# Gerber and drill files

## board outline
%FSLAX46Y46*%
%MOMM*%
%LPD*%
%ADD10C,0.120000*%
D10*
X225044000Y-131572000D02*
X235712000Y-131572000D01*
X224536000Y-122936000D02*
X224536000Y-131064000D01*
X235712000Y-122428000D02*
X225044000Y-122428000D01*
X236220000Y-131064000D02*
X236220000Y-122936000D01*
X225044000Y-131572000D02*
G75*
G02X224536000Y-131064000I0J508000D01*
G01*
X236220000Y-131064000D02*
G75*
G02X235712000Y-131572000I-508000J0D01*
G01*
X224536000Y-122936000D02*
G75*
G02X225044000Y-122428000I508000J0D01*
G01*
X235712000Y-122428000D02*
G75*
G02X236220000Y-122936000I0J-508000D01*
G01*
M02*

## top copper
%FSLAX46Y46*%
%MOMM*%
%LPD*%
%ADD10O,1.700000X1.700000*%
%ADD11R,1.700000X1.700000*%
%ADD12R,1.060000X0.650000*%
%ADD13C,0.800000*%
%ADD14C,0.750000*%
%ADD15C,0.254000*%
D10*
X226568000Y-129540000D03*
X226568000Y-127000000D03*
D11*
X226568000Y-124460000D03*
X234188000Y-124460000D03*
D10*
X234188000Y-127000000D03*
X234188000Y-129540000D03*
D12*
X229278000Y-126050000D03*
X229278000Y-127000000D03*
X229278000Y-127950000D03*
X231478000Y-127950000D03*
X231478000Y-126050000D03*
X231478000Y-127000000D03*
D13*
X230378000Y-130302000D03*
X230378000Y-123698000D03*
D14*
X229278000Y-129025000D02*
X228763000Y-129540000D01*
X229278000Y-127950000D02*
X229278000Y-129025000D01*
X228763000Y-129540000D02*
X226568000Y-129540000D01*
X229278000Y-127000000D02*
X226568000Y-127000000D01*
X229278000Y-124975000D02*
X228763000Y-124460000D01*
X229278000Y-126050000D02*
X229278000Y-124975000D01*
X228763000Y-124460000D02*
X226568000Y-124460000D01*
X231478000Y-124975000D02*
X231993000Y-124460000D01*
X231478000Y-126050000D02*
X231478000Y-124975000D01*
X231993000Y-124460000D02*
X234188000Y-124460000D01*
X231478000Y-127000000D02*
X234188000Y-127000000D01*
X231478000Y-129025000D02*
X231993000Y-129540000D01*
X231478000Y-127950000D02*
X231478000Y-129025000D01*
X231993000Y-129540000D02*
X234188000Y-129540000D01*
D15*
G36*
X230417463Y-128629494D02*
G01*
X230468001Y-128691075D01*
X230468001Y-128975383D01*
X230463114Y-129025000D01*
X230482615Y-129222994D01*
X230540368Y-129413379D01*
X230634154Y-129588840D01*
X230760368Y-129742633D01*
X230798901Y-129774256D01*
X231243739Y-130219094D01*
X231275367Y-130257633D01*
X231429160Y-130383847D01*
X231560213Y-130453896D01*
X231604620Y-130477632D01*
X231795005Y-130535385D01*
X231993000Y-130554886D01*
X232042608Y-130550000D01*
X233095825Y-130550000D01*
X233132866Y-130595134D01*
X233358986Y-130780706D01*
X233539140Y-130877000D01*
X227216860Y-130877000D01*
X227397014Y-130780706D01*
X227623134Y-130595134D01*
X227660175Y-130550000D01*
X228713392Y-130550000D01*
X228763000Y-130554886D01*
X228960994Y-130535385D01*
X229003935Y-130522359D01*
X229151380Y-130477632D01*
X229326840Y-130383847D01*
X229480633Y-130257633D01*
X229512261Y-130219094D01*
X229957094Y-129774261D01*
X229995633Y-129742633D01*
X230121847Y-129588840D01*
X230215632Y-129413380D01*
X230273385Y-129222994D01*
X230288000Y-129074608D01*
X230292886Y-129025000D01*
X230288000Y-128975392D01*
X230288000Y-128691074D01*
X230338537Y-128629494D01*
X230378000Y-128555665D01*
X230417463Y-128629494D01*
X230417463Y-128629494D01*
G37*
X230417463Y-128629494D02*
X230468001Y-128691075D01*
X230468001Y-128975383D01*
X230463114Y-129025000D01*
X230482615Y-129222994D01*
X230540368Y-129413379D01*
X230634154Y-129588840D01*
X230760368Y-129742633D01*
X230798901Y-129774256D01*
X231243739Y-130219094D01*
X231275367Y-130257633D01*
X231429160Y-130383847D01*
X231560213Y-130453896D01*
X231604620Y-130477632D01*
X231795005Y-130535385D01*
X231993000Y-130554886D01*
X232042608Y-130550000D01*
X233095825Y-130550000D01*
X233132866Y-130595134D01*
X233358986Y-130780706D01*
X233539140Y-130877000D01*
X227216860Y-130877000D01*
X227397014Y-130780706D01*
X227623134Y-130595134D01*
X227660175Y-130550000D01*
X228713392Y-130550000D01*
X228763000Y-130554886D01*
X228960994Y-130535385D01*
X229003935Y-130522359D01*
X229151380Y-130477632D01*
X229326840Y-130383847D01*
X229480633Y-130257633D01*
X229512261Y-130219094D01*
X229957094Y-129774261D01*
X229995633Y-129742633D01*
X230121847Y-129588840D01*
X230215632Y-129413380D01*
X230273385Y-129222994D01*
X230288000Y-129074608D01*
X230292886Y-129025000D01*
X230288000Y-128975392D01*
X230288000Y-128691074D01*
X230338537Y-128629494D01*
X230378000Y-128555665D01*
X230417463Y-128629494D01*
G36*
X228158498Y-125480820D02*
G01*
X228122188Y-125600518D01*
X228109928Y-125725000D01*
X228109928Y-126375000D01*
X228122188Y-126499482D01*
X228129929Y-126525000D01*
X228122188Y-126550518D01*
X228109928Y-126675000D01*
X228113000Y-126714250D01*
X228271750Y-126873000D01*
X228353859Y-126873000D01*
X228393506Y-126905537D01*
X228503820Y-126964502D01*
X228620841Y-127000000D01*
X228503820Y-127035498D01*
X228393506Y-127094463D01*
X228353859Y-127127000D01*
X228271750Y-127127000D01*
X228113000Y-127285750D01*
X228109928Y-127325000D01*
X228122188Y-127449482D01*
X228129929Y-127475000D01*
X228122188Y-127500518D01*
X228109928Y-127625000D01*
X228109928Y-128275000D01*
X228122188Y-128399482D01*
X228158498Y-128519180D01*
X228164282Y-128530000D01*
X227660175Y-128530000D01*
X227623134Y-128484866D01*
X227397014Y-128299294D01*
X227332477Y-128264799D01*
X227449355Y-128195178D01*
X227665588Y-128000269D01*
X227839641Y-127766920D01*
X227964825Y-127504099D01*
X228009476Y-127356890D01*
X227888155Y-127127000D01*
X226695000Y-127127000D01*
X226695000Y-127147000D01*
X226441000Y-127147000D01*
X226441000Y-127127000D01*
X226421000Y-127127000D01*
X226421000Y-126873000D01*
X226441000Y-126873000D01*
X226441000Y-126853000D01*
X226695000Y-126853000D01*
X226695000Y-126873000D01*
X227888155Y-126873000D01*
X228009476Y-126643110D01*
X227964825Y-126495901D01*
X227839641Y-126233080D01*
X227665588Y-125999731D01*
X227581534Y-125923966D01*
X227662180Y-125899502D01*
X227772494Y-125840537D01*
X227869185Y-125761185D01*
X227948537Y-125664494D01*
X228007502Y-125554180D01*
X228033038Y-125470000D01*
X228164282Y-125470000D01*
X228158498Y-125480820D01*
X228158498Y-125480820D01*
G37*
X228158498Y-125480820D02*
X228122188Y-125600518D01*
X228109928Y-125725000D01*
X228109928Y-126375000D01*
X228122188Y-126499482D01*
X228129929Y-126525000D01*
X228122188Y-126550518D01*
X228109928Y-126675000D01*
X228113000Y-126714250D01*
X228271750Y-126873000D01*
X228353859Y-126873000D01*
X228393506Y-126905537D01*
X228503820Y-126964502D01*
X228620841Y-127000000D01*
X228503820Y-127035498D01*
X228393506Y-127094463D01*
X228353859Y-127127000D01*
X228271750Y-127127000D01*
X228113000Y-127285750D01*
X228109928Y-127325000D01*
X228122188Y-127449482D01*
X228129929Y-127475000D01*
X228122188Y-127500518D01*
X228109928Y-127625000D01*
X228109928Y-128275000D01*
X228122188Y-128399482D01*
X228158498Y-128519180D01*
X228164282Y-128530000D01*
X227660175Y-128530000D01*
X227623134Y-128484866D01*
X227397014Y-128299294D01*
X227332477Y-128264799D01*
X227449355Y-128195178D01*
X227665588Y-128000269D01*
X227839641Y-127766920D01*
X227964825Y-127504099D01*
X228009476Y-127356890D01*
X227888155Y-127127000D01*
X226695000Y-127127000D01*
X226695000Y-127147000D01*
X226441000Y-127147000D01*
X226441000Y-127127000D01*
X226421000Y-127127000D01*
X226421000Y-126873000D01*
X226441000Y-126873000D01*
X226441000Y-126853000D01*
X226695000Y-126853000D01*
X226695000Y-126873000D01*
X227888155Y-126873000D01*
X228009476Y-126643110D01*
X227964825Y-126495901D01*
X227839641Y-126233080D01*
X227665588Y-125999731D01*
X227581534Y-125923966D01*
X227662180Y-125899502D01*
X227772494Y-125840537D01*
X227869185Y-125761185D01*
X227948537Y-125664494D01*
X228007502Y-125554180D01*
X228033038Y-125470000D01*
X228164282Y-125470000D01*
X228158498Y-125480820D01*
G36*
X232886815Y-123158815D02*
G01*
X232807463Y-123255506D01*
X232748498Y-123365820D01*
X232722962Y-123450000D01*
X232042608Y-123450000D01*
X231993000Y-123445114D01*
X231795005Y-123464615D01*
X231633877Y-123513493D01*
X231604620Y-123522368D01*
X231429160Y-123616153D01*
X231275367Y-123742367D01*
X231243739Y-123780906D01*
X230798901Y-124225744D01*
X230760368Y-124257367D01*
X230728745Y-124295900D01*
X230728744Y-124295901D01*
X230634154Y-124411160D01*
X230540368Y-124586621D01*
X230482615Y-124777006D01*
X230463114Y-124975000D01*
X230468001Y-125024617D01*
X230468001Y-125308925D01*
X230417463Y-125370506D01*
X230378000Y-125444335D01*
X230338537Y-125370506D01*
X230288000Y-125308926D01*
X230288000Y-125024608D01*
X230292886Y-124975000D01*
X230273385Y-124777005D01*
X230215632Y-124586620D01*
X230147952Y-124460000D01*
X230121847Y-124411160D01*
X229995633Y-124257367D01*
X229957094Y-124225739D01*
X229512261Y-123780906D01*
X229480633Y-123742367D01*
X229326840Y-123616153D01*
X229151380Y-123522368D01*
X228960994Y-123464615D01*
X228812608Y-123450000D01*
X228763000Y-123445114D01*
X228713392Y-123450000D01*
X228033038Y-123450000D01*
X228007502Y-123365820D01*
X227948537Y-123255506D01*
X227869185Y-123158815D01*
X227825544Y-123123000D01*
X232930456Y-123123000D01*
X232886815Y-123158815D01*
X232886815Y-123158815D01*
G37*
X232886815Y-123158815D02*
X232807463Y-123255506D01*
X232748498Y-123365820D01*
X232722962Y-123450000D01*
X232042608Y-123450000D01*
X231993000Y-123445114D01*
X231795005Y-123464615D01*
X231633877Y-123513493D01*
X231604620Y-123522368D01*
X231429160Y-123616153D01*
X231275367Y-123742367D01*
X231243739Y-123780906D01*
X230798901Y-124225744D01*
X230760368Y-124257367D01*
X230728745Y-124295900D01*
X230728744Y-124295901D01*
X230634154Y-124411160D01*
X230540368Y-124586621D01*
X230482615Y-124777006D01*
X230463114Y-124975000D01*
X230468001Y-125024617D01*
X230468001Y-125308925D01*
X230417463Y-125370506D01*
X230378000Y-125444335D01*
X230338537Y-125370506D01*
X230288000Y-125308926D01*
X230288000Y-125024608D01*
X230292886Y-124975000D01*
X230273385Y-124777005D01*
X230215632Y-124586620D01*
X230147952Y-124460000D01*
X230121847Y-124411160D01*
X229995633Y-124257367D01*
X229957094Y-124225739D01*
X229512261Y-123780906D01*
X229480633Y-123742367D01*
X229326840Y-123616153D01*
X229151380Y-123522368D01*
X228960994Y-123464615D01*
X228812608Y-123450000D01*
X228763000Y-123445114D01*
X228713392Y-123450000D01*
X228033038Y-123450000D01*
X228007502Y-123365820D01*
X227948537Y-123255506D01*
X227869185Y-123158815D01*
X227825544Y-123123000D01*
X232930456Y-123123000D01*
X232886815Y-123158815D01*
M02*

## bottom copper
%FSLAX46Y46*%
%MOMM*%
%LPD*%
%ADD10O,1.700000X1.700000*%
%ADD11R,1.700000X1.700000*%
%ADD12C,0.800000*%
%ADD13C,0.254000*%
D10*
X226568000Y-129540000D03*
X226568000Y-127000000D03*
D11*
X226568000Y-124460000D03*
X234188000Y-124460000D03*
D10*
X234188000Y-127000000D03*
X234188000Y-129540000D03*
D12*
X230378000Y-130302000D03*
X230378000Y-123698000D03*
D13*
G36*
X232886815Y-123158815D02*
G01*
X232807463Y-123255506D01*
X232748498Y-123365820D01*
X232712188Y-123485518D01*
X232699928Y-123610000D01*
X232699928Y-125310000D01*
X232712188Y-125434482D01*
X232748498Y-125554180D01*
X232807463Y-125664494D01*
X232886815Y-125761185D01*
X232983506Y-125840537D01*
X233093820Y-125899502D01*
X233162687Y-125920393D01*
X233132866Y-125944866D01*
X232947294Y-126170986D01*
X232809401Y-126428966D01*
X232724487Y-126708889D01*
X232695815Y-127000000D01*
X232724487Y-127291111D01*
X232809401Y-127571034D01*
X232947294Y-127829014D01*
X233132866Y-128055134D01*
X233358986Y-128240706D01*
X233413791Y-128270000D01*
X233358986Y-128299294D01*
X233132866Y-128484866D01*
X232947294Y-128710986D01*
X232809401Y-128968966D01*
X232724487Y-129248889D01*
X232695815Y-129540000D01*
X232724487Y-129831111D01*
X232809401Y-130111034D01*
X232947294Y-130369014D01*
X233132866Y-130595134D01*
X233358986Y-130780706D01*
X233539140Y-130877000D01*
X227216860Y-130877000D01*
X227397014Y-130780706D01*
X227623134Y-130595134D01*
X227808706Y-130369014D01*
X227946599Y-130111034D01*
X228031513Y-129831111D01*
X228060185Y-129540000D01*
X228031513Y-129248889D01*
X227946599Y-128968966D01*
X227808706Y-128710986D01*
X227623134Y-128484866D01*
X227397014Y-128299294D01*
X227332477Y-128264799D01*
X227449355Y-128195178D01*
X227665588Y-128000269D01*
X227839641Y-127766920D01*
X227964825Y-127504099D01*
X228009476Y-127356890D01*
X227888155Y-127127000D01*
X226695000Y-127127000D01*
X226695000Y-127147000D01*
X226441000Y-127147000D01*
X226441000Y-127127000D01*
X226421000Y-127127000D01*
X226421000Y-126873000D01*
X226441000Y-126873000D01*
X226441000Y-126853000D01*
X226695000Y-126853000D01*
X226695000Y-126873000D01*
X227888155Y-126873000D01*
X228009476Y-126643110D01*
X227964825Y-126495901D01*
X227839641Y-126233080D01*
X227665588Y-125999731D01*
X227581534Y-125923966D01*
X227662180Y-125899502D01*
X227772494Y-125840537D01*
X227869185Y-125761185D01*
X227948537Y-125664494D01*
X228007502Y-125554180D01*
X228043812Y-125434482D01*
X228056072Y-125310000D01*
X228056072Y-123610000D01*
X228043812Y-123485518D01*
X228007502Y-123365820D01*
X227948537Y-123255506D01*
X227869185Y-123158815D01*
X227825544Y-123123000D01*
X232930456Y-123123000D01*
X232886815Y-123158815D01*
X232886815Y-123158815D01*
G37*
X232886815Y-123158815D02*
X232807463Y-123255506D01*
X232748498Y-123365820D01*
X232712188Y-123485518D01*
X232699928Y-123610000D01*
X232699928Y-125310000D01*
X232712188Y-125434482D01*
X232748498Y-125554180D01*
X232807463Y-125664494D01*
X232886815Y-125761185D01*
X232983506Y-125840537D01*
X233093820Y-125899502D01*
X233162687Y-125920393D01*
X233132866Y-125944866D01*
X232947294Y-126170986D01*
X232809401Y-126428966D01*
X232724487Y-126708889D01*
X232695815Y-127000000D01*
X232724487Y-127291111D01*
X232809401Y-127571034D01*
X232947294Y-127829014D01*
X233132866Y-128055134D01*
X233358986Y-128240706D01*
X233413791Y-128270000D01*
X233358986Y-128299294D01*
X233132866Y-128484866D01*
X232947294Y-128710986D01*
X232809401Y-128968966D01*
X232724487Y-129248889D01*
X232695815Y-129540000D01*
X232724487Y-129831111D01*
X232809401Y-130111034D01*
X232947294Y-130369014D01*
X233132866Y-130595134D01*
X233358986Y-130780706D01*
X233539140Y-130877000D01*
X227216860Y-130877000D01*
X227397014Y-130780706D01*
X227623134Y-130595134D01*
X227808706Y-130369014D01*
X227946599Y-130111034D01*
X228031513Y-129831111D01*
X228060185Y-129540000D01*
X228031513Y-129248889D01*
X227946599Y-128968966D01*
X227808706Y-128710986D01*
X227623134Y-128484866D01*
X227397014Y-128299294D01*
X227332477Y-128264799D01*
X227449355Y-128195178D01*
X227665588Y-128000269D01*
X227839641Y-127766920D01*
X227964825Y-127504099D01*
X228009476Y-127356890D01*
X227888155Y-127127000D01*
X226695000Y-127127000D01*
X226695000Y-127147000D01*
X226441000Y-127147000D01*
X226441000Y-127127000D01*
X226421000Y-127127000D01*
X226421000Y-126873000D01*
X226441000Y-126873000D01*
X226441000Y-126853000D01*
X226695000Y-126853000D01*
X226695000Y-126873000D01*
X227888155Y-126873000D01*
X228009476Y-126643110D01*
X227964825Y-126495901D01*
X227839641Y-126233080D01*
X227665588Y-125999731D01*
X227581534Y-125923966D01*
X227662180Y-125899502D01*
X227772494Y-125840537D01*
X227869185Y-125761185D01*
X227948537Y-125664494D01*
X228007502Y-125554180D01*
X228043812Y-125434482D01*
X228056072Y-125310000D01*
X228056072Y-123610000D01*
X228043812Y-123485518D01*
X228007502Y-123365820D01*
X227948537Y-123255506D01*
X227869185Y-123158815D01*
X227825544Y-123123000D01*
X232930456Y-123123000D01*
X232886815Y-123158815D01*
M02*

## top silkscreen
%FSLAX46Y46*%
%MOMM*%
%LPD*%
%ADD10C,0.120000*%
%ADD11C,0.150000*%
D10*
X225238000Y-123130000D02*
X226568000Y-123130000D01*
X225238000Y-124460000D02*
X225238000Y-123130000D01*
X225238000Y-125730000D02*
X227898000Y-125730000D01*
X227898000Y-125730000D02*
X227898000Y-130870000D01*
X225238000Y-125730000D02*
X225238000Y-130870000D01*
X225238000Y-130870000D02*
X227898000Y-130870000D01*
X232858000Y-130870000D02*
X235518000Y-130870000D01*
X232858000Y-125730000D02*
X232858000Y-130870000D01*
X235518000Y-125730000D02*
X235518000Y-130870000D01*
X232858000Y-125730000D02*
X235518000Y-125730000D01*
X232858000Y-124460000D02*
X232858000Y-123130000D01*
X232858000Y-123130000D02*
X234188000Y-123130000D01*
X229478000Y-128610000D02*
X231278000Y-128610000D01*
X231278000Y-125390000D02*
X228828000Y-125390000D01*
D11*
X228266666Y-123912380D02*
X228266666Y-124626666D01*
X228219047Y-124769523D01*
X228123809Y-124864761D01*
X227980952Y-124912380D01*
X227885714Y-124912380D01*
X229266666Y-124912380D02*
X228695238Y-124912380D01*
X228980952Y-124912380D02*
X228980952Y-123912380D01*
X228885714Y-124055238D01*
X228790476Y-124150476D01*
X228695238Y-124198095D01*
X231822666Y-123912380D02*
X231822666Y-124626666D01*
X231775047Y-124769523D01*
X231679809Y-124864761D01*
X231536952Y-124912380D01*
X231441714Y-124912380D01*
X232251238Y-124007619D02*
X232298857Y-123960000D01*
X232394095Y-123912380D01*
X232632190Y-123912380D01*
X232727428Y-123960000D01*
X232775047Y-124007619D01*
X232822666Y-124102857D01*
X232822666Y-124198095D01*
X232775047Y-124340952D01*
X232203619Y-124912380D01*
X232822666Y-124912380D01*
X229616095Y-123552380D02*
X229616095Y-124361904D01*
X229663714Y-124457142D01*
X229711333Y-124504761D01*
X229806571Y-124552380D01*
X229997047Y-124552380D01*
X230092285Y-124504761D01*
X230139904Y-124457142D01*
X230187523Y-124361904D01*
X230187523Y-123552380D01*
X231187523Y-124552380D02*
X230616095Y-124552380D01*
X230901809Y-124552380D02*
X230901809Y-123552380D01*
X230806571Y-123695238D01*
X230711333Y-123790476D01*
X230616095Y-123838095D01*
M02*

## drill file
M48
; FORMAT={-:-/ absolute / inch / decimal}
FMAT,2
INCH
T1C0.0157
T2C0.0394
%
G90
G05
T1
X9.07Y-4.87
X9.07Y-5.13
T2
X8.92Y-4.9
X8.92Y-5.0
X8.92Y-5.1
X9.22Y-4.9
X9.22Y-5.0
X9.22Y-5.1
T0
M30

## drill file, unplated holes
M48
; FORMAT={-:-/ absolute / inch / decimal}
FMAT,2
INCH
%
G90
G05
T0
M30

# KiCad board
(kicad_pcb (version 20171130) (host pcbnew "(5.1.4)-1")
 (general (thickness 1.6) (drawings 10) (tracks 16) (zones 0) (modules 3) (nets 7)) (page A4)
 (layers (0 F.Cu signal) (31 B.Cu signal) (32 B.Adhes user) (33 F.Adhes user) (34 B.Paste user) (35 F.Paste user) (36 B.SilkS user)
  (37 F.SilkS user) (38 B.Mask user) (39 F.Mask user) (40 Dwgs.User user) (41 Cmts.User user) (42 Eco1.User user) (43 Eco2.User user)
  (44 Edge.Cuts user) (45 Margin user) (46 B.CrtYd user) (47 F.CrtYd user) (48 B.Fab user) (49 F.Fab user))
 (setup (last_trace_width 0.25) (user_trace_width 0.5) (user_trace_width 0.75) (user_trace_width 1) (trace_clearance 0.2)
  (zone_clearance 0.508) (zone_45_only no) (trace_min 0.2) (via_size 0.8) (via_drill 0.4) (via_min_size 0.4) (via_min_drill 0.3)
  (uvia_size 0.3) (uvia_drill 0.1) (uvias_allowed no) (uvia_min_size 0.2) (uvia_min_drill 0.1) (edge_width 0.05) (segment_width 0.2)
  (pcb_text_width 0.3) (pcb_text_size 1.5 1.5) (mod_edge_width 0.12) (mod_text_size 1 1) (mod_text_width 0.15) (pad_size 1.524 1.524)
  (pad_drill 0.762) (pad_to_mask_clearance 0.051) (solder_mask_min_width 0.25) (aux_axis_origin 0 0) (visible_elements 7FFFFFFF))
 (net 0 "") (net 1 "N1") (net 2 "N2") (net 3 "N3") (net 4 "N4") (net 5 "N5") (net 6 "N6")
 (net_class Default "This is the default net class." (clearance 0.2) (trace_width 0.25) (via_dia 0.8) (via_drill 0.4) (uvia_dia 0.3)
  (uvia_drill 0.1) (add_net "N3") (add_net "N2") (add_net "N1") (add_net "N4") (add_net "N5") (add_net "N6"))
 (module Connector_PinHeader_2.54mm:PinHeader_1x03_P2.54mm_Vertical (layer F.Cu) (at 226.568 124.46)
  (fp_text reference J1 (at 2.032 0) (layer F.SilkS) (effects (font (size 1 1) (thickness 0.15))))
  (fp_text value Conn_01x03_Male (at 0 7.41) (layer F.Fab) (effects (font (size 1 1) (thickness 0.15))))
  (fp_line (start -1.33 -1.33) (end 0 -1.33) (layer F.SilkS) (width 0.12))
  (fp_line (start -1.33 0) (end -1.33 -1.33) (layer F.SilkS) (width 0.12))
  (fp_line (start -1.33 1.27) (end 1.33 1.27) (layer F.SilkS) (width 0.12))
  (fp_line (start 1.33 1.27) (end 1.33 6.41) (layer F.SilkS) (width 0.12))
  (fp_line (start -1.33 1.27) (end -1.33 6.41) (layer F.SilkS) (width 0.12))
  (fp_line (start -1.33 6.41) (end 1.33 6.41) (layer F.SilkS) (width 0.12))
  (pad 3 thru_hole oval (at 0 5.08) (size 1.7 1.7) (drill 1) (layers *.Cu *.Mask) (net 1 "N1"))
  (pad 2 thru_hole oval (at 0 2.54) (size 1.7 1.7) (drill 1) (layers *.Cu *.Mask) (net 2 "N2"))
  (pad 1 thru_hole rect (at 0 0) (size 1.7 1.7) (drill 1) (layers *.Cu *.Mask) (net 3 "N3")))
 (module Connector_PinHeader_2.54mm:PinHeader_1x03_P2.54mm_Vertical (layer F.Cu) (at 234.188 124.46)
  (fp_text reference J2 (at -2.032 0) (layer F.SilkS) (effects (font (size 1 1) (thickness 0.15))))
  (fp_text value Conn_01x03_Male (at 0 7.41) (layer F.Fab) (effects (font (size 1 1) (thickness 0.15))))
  (fp_line (start -1.33 6.41) (end 1.33 6.41) (layer F.SilkS) (width 0.12))
  (fp_line (start -1.33 1.27) (end -1.33 6.41) (layer F.SilkS) (width 0.12))
  (fp_line (start 1.33 1.27) (end 1.33 6.41) (layer F.SilkS) (width 0.12))
  (fp_line (start -1.33 1.27) (end 1.33 1.27) (layer F.SilkS) (width 0.12))
  (fp_line (start -1.33 0) (end -1.33 -1.33) (layer F.SilkS) (width 0.12))
  (fp_line (start -1.33 -1.33) (end 0 -1.33) (layer F.SilkS) (width 0.12))
  (pad 1 thru_hole rect (at 0 0) (size 1.7 1.7) (drill 1) (layers *.Cu *.Mask) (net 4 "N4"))
  (pad 2 thru_hole oval (at 0 2.54) (size 1.7 1.7) (drill 1) (layers *.Cu *.Mask) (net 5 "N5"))
  (pad 3 thru_hole oval (at 0 5.08) (size 1.7 1.7) (drill 1) (layers *.Cu *.Mask) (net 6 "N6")))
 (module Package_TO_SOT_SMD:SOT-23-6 (layer F.Cu) (at 230.378 127)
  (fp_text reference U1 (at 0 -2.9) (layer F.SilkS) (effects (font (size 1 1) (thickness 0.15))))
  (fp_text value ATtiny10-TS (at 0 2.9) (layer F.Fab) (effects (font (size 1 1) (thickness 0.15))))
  (fp_line (start -0.9 1.61) (end 0.9 1.61) (layer F.SilkS) (width 0.12))
  (fp_line (start 0.9 -1.61) (end -1.55 -1.61) (layer F.SilkS) (width 0.12))
  (pad 1 smd rect (at -1.1 -0.95) (size 1.06 0.65) (layers F.Cu F.Paste F.Mask) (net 3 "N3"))
  (pad 2 smd rect (at -1.1 0) (size 1.06 0.65) (layers F.Cu F.Paste F.Mask) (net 2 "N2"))
  (pad 3 smd rect (at -1.1 0.95) (size 1.06 0.65) (layers F.Cu F.Paste F.Mask) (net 1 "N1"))
  (pad 4 smd rect (at 1.1 0.95) (size 1.06 0.65) (layers F.Cu F.Paste F.Mask) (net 6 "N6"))
  (pad 6 smd rect (at 1.1 -0.95) (size 1.06 0.65) (layers F.Cu F.Paste F.Mask) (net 4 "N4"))
  (pad 5 smd rect (at 1.1 0) (size 1.06 0.65) (layers F.Cu F.Paste F.Mask) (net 5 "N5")))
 (gr_line (start 225.044 131.572) (end 235.712 131.572) (layer Edge.Cuts) (width 0.12))
 (gr_line (start 224.536 122.936) (end 224.536 131.064) (layer Edge.Cuts) (width 0.12))
 (gr_line (start 235.712 122.428) (end 225.044 122.428) (layer Edge.Cuts) (width 0.12))
 (gr_line (start 236.22 131.064) (end 236.22 122.936) (layer Edge.Cuts) (width 0.12))
 (gr_arc (start 225.044 131.064) (end 224.536 131.064) (angle -90) (layer Edge.Cuts) (width 0.12))
 (gr_arc (start 235.712 131.064) (end 235.712 131.572) (angle -90) (layer Edge.Cuts) (width 0.12))
 (gr_arc (start 225.044 122.936) (end 225.044 122.428) (angle -90) (layer Edge.Cuts) (width 0.12))
 (gr_arc (start 235.712 122.936) (end 236.22 122.936) (angle -90) (layer Edge.Cuts) (width 0.12))
 (segment (start 229.278 129.025) (end 228.763 129.54) (width 0.75) (layer F.Cu) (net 1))
 (segment (start 229.278 127.95) (end 229.278 129.025) (width 0.75) (layer F.Cu) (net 1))
 (segment (start 228.763 129.54) (end 226.568 129.54) (width 0.75) (layer F.Cu) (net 1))
 (segment (start 229.278 127) (end 226.568 127) (width 0.75) (layer F.Cu) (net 2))
 (via (at 230.378 130.302) (size 0.8) (drill 0.4) (layers F.Cu B.Cu) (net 2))
 (via (at 230.378 123.698) (size 0.8) (drill 0.4) (layers F.Cu B.Cu) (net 2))
 (segment (start 229.278 124.975) (end 228.763 124.46) (width 0.75) (layer F.Cu) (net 3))
 (segment (start 229.278 126.05) (end 229.278 124.975) (width 0.75) (layer F.Cu) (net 3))
 (segment (start 228.763 124.46) (end 226.568 124.46) (width 0.75) (layer F.Cu) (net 3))
 (segment (start 231.478 124.975) (end 231.993 124.46) (width 0.75) (layer F.Cu) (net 4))
 (segment (start 231.478 126.05) (end 231.478 124.975) (width 0.75) (layer F.Cu) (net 4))
 (segment (start 231.993 124.46) (end 234.188 124.46) (width 0.75) (layer F.Cu) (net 4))
 (segment (start 231.478 127) (end 234.188 127) (width 0.75) (layer F.Cu) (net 5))
 (segment (start 231.478 129.025) (end 231.993 129.54) (width 0.75) (layer F.Cu) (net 6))
 (segment (start 231.478 127.95) (end 231.478 129.025) (width 0.75) (layer F.Cu) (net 6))
 (segment (start 231.993 129.54) (end 234.188 129.54) (width 0.75) (layer F.Cu) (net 6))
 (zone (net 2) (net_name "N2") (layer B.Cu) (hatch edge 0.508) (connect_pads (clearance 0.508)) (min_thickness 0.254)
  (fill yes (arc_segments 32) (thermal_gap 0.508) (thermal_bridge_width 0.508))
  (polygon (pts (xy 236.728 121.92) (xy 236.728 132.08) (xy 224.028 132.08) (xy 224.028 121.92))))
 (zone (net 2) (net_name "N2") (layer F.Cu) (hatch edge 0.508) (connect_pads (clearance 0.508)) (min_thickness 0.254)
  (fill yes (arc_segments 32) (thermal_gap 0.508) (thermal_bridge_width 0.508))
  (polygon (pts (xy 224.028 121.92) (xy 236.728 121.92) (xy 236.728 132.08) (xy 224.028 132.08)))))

